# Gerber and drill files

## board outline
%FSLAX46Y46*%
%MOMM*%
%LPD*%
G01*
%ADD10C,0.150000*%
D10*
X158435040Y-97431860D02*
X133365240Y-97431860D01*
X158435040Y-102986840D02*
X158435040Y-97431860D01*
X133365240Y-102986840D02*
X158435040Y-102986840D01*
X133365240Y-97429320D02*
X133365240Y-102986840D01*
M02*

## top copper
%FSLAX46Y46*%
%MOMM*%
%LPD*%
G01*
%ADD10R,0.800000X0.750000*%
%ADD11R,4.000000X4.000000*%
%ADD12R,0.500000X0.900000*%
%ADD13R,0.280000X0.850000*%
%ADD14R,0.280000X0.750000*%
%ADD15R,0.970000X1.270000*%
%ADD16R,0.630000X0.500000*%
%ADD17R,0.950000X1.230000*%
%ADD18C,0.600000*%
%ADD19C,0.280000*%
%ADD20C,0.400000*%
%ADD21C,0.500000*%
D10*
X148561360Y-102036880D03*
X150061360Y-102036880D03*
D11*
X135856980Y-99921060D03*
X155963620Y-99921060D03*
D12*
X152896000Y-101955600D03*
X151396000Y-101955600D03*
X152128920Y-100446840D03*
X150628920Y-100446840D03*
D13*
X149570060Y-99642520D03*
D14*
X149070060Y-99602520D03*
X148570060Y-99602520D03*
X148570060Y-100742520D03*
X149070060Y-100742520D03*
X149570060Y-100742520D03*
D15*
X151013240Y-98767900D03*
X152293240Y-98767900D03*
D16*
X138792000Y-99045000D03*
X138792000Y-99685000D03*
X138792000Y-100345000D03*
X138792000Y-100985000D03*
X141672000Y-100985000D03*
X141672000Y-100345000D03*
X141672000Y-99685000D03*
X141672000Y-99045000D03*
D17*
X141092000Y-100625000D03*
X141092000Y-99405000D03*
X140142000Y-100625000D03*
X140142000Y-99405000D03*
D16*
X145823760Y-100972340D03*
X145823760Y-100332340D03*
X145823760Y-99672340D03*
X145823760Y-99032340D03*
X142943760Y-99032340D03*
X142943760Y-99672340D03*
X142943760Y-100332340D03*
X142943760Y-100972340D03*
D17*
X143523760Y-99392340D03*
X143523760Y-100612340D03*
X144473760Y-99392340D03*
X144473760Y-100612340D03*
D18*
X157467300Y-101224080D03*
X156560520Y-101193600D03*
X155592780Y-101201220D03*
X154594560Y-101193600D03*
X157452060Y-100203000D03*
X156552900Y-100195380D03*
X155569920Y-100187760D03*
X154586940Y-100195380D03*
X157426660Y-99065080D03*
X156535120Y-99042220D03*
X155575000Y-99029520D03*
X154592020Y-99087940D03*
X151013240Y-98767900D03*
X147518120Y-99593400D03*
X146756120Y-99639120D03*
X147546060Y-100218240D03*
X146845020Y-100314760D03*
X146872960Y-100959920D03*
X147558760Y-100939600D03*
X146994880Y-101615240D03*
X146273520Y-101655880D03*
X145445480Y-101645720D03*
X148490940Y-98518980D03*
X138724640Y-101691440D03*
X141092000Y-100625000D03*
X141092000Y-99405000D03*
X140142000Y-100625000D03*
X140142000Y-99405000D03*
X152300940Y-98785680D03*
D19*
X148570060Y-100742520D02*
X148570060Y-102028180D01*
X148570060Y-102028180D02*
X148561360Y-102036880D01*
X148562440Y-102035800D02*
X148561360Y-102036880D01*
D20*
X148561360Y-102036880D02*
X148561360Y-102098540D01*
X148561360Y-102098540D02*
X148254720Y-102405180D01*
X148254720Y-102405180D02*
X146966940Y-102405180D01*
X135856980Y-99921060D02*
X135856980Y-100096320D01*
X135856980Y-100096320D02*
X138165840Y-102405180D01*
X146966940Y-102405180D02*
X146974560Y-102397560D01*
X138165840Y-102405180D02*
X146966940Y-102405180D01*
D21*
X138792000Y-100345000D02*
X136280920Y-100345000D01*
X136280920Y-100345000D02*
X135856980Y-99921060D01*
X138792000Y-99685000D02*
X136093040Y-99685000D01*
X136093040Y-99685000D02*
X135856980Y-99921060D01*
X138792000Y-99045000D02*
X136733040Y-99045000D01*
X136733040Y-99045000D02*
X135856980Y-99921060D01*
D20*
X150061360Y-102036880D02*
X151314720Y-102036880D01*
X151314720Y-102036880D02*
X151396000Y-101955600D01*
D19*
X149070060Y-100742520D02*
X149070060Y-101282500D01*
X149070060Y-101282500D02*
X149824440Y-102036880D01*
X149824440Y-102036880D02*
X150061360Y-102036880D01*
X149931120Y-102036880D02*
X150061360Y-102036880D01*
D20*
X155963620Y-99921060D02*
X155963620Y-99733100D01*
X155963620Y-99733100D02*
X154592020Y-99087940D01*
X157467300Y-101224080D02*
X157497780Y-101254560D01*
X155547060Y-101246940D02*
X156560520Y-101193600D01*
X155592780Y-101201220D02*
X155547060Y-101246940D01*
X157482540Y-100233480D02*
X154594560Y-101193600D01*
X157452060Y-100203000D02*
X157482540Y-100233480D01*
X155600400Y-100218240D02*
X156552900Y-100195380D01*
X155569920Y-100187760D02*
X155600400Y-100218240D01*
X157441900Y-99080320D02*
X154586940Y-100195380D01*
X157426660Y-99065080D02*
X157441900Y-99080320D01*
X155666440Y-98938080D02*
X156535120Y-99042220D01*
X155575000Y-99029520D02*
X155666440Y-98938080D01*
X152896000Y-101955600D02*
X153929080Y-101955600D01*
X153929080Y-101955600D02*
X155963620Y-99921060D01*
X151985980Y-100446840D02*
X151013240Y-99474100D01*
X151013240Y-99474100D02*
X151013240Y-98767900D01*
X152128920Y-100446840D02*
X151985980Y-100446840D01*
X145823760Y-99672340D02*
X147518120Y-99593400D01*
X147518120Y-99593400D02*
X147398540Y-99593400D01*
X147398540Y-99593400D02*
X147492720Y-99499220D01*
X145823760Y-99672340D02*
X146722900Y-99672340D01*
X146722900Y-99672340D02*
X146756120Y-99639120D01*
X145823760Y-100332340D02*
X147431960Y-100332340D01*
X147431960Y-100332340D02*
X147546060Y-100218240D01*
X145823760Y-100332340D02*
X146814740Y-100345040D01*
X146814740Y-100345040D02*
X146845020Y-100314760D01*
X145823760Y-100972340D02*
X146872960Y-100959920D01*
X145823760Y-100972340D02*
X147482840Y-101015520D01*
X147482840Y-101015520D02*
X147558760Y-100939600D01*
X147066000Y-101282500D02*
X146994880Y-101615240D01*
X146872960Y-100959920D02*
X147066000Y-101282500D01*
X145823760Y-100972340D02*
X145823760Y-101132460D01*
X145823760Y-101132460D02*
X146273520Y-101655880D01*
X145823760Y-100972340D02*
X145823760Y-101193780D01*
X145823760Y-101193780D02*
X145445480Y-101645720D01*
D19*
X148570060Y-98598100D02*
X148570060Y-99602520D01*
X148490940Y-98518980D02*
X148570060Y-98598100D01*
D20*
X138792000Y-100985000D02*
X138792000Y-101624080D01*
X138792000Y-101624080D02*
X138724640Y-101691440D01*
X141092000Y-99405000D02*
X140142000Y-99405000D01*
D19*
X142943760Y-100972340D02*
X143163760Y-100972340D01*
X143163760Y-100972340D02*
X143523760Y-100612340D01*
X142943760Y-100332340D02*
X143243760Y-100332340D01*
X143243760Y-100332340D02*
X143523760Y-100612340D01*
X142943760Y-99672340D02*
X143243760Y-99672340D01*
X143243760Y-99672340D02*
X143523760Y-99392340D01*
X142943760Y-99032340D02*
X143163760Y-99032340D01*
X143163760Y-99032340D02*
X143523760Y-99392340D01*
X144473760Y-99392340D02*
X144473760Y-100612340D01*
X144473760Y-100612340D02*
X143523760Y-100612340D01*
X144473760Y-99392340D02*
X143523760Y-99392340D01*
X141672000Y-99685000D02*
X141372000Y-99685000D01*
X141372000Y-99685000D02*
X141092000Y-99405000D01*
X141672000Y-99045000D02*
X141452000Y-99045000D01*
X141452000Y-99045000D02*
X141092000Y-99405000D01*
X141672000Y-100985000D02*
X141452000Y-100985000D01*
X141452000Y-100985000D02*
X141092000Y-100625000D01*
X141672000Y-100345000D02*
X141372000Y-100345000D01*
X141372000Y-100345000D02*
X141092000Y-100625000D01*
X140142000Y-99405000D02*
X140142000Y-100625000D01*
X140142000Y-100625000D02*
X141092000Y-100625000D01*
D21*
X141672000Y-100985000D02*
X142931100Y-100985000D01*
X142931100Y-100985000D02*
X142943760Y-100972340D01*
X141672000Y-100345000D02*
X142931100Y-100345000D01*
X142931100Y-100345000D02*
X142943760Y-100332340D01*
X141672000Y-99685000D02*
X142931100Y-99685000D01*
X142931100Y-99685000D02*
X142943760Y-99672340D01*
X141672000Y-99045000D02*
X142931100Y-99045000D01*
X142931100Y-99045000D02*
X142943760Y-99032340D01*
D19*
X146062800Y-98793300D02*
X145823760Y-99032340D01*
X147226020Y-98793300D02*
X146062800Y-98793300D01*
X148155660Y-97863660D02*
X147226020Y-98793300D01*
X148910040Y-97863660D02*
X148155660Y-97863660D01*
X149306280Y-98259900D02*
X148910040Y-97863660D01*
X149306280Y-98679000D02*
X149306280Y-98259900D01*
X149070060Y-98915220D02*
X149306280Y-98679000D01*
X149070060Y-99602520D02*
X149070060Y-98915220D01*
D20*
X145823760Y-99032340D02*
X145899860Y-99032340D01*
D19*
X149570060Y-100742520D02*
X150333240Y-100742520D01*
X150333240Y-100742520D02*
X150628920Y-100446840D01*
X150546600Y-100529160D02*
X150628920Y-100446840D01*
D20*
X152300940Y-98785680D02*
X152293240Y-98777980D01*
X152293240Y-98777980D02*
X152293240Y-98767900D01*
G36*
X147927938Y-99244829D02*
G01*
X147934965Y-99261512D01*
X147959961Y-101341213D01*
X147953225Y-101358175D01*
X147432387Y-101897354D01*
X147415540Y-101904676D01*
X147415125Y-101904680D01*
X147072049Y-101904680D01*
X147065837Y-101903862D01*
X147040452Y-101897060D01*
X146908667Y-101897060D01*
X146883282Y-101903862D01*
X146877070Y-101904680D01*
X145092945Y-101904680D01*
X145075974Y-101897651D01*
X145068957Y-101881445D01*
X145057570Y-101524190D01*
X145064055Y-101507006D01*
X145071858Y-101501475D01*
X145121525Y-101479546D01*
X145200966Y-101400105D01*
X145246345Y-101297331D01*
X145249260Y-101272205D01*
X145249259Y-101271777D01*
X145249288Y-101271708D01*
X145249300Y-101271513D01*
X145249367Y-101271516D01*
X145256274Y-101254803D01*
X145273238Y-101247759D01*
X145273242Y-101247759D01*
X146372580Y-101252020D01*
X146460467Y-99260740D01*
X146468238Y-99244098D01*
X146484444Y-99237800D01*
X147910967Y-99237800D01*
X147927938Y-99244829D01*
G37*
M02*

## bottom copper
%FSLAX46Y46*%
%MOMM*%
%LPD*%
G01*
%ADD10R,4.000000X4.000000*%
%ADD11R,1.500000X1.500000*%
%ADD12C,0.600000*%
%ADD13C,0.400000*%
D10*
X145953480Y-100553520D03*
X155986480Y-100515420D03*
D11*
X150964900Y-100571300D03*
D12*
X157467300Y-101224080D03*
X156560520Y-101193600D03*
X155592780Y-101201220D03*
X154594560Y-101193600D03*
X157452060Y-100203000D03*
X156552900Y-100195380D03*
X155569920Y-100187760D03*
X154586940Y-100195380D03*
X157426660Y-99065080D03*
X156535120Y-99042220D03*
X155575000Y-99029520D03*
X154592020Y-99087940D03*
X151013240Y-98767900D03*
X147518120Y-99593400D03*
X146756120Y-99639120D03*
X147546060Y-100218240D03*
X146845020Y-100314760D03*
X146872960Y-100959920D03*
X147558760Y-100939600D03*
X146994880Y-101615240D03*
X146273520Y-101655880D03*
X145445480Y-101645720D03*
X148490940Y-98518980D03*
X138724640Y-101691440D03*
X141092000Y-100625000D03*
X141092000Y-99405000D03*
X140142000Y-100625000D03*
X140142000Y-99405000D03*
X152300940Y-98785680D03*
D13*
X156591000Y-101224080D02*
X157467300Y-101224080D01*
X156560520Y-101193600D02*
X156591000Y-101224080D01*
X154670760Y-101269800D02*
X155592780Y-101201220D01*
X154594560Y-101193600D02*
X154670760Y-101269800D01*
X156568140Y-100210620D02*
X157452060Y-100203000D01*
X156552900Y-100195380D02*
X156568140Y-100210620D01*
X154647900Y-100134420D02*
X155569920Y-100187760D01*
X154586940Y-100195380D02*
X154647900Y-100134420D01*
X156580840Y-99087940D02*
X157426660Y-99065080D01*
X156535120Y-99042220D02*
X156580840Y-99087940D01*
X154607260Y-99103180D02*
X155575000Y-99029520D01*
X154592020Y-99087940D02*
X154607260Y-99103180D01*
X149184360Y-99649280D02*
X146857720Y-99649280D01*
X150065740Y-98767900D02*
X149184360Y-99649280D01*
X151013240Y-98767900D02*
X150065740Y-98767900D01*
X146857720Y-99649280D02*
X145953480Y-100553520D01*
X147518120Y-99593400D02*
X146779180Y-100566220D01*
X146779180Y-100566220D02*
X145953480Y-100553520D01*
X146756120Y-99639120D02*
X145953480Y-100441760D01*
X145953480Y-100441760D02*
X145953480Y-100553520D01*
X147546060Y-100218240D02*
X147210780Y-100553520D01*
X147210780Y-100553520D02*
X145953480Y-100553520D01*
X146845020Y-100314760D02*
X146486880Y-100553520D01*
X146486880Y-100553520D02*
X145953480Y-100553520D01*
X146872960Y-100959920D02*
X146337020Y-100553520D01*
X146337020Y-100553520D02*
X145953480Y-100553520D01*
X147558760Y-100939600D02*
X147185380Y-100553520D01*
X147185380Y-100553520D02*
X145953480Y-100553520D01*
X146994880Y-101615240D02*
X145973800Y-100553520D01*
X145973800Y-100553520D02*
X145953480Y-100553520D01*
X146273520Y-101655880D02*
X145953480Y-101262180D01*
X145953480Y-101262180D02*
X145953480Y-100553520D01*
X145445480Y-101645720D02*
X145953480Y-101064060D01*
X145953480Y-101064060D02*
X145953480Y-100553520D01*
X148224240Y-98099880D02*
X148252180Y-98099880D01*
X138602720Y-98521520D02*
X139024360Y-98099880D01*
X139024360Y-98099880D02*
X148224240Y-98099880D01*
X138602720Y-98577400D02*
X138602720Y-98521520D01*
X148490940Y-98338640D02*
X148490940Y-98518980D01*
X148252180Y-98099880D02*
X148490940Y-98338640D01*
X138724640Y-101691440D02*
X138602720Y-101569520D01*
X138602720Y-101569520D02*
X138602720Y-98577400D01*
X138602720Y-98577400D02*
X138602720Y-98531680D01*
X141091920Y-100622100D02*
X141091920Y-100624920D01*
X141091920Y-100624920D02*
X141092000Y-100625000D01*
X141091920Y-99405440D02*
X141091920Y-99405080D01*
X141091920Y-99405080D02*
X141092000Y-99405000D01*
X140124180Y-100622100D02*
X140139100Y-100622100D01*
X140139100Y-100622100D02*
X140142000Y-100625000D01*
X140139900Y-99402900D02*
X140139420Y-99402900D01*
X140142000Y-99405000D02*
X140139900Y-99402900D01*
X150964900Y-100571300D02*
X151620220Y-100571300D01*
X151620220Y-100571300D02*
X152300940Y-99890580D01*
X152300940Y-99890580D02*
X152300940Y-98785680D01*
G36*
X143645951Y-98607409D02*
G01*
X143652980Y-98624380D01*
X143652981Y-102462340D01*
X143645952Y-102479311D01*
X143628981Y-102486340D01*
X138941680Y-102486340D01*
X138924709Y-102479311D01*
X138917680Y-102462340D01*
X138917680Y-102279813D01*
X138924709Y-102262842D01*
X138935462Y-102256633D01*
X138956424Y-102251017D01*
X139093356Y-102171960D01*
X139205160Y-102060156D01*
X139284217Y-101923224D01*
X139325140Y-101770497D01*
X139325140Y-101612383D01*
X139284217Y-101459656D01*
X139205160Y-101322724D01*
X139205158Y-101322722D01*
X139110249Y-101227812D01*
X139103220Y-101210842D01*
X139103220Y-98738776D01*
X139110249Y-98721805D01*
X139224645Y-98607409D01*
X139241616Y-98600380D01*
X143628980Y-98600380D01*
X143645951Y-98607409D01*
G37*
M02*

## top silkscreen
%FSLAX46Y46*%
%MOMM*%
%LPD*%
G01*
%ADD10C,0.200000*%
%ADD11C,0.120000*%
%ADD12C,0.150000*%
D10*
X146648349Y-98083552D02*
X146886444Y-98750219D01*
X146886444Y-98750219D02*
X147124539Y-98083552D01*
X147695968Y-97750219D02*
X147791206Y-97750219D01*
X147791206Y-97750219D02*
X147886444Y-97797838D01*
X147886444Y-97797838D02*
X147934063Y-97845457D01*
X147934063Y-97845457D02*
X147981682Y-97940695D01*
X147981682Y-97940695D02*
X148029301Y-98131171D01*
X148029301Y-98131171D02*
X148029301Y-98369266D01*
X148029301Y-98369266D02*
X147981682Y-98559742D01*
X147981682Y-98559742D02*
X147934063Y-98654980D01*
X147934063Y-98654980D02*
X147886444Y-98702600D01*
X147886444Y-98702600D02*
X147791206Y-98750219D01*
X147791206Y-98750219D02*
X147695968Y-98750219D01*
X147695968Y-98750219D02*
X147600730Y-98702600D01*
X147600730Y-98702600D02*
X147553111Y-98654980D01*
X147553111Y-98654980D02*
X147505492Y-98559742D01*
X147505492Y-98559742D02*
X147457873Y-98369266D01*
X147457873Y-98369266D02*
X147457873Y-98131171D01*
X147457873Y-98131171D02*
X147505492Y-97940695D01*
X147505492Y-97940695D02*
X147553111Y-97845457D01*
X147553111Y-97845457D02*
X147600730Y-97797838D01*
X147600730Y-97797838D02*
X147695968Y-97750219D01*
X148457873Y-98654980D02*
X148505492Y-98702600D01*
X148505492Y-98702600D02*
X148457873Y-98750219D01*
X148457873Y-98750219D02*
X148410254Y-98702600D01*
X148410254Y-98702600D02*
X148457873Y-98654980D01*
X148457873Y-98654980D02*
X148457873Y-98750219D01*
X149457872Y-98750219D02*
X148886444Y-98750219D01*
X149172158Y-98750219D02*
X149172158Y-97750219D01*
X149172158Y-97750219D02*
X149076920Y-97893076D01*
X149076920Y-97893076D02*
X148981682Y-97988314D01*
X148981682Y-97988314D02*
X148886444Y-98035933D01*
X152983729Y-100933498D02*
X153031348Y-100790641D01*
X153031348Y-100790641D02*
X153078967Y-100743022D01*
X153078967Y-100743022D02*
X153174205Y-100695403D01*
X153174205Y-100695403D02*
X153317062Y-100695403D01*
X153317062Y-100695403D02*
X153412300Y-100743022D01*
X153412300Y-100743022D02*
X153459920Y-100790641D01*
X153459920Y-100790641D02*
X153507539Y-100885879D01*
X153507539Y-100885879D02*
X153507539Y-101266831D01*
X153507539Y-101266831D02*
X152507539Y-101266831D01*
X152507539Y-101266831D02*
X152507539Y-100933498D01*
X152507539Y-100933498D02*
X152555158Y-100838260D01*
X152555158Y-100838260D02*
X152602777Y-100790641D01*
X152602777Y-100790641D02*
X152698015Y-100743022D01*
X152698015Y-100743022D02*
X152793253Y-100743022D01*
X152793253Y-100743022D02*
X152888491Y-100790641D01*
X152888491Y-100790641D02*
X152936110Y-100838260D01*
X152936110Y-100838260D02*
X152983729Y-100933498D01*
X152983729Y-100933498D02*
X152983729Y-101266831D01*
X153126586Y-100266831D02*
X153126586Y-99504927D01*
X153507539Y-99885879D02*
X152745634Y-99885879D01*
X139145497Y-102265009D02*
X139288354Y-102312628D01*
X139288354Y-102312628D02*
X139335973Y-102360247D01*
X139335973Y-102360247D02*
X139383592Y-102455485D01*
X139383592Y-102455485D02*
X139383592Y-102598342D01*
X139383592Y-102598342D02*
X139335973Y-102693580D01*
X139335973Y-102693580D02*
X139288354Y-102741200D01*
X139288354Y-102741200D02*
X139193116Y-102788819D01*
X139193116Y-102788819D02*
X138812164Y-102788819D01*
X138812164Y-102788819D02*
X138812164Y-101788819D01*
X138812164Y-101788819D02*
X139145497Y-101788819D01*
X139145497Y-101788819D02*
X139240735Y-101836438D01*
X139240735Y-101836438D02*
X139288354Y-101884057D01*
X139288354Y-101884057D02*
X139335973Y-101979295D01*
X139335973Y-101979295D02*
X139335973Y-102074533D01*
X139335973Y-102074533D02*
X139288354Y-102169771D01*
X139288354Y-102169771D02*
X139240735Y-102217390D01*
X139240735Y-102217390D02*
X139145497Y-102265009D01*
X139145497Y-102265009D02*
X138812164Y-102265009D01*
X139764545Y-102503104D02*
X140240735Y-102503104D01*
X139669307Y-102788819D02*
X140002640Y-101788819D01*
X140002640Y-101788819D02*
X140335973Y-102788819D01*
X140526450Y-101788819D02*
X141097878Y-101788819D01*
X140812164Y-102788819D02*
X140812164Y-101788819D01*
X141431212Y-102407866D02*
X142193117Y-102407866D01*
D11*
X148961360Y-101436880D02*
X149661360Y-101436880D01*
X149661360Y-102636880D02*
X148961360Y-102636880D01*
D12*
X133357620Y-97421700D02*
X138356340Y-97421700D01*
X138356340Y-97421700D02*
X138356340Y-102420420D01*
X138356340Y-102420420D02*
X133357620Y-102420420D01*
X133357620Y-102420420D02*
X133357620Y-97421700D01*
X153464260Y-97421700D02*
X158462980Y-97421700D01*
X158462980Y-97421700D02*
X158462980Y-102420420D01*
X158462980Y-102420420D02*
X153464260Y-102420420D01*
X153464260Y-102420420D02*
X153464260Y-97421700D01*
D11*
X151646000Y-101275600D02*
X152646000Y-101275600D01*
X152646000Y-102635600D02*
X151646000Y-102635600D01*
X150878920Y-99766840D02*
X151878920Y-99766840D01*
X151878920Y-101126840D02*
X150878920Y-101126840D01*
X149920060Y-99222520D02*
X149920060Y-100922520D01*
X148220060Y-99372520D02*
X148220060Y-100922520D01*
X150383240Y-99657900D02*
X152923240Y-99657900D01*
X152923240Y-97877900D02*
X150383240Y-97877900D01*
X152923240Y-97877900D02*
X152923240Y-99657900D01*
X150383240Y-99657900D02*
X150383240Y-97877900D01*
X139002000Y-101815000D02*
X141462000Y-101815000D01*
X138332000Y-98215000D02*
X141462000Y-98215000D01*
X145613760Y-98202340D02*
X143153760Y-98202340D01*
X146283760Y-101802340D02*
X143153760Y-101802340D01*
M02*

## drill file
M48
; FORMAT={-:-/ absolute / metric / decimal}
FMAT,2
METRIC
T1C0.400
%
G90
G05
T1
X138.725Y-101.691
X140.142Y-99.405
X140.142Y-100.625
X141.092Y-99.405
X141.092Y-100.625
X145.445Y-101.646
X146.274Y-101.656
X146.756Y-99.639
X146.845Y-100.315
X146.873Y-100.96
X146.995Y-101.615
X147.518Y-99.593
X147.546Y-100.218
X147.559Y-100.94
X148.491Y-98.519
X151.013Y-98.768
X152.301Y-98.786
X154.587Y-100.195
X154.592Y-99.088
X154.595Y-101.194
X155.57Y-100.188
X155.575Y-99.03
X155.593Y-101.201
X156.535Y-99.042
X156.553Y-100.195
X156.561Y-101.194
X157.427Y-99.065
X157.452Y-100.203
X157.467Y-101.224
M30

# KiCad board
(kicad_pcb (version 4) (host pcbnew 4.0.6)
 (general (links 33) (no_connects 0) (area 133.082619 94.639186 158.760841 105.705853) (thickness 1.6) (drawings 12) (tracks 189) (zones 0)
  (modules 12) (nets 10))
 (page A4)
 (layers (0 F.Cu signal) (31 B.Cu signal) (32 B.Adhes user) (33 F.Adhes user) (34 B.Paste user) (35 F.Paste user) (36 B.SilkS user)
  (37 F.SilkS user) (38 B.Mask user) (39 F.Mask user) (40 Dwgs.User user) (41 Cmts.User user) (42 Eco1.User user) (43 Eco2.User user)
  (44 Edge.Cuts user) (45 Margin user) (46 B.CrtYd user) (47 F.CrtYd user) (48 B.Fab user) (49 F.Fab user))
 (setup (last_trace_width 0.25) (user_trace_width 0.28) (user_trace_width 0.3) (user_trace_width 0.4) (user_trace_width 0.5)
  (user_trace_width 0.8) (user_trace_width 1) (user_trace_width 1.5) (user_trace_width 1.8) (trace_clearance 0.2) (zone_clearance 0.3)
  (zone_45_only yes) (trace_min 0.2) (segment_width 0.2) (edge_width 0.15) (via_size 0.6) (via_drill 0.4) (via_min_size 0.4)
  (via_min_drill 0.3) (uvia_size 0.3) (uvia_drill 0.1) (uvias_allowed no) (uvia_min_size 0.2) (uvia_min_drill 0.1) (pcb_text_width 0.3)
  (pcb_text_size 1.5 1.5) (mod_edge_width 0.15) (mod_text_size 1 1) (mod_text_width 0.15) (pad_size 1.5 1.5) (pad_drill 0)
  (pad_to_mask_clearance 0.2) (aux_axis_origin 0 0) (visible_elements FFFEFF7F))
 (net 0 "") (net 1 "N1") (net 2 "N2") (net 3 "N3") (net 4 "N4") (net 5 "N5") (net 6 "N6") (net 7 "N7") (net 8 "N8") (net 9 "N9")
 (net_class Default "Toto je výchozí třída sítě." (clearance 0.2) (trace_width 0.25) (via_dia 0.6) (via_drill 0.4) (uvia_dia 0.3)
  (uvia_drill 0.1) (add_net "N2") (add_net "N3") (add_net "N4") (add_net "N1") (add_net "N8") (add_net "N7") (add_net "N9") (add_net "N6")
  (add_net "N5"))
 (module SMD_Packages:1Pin (layer B.Cu) (at 145.95348 100.55352)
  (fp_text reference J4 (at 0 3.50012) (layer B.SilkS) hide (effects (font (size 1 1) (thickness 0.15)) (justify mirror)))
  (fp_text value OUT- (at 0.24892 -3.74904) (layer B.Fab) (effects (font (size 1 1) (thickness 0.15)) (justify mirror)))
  (pad 1 smd rect (at 0 0) (size 4 4) (layers B.Cu B.Paste B.Mask) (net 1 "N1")))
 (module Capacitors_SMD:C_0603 (layer F.Cu) (at 149.31136 102.03688)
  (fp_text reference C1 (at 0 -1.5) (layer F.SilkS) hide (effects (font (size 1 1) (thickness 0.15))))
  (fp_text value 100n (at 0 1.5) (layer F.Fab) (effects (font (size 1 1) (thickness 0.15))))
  (fp_line (start -0.35 -0.6) (end 0.35 -0.6) (layer F.SilkS) (width 0.12))
  (fp_line (start 0.35 0.6) (end -0.35 0.6) (layer F.SilkS) (width 0.12))
  (pad 1 smd rect (at -0.75 0) (size 0.8 0.75) (layers F.Cu F.Paste F.Mask) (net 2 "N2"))
  (pad 2 smd rect (at 0.75 0) (size 0.8 0.75) (layers F.Cu F.Paste F.Mask) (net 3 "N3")))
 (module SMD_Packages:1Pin (layer F.Cu) (at 135.85698 99.92106)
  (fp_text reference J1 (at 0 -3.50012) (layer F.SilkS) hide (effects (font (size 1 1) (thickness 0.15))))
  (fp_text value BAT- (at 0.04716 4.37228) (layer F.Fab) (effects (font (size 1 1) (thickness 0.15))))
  (fp_line (start -2.49936 -2.49936) (end 2.49936 -2.49936) (layer F.SilkS) (width 0.15))
  (fp_line (start 2.49936 -2.49936) (end 2.49936 2.49936) (layer F.SilkS) (width 0.15))
  (fp_line (start 2.49936 2.49936) (end -2.49936 2.49936) (layer F.SilkS) (width 0.15))
  (fp_line (start -2.49936 2.49936) (end -2.49936 -2.49936) (layer F.SilkS) (width 0.15))
  (pad 1 smd rect (at 0 0) (size 4 4) (layers F.Cu F.Paste F.Mask) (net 2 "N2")))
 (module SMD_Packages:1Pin (layer F.Cu) (at 155.96362 99.92106)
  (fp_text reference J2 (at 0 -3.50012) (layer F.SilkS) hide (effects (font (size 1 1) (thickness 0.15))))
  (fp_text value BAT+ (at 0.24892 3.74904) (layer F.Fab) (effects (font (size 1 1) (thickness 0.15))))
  (fp_line (start -2.49936 -2.49936) (end 2.49936 -2.49936) (layer F.SilkS) (width 0.15))
  (fp_line (start 2.49936 -2.49936) (end 2.49936 2.49936) (layer F.SilkS) (width 0.15))
  (fp_line (start 2.49936 2.49936) (end -2.49936 2.49936) (layer F.SilkS) (width 0.15))
  (fp_line (start -2.49936 2.49936) (end -2.49936 -2.49936) (layer F.SilkS) (width 0.15))
  (pad 1 smd rect (at 0 0) (size 4 4) (layers F.Cu F.Paste F.Mask) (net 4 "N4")))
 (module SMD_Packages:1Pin (layer B.Cu) (at 155.98648 100.51542)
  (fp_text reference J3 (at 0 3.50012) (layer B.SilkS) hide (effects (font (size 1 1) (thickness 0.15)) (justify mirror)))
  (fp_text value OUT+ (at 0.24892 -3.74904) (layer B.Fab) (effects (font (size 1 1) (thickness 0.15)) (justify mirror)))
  (pad 1 smd rect (at 0 0) (size 4 4) (layers B.Cu B.Paste B.Mask) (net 4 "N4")))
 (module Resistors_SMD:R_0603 (layer F.Cu) (at 152.146 101.9556 180)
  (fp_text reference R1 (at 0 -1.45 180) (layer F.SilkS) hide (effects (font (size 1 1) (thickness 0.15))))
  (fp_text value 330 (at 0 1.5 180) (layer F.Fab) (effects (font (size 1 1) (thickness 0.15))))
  (fp_line (start 0.5 0.68) (end -0.5 0.68) (layer F.SilkS) (width 0.12))
  (fp_line (start -0.5 -0.68) (end 0.5 -0.68) (layer F.SilkS) (width 0.12))
  (pad 1 smd rect (at -0.75 0 180) (size 0.5 0.9) (layers F.Cu F.Paste F.Mask) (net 4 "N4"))
  (pad 2 smd rect (at 0.75 0 180) (size 0.5 0.9) (layers F.Cu F.Paste F.Mask) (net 3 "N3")))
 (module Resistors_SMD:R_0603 (layer F.Cu) (at 151.37892 100.44684 180)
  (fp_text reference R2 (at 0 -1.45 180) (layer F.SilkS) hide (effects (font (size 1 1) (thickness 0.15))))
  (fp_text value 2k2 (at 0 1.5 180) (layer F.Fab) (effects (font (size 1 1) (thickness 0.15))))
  (fp_line (start 0.5 0.68) (end -0.5 0.68) (layer F.SilkS) (width 0.12))
  (fp_line (start -0.5 -0.68) (end 0.5 -0.68) (layer F.SilkS) (width 0.12))
  (pad 1 smd rect (at -0.75 0 180) (size 0.5 0.9) (layers F.Cu F.Paste F.Mask) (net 1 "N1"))
  (pad 2 smd rect (at 0.75 0 180) (size 0.5 0.9) (layers F.Cu F.Paste F.Mask) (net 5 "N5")))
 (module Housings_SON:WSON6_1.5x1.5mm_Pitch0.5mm (layer F.Cu) (at 149.07006 100.17252 270)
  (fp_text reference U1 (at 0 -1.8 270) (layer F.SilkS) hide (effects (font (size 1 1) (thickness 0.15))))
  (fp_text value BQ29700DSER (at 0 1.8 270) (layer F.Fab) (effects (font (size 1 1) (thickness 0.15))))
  (fp_line (start -0.95 -0.85) (end 0.75 -0.85) (layer F.SilkS) (width 0.12))
  (fp_line (start -0.8 0.85) (end 0.75 0.85) (layer F.SilkS) (width 0.12))
  (pad 1 smd rect (at -0.53 -0.5 180) (size 0.28 0.85) (layers F.Cu F.Paste F.Mask))
  (pad 2 smd rect (at -0.57 0 180) (size 0.28 0.75) (layers F.Cu F.Paste F.Mask) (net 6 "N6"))
  (pad 3 smd rect (at -0.57 0.5 180) (size 0.28 0.75) (layers F.Cu F.Paste F.Mask) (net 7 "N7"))
  (pad 4 smd rect (at 0.57 0.5 180) (size 0.28 0.75) (layers F.Cu F.Paste F.Mask) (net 2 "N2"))
  (pad 5 smd rect (at 0.57 0 180) (size 0.28 0.75) (layers F.Cu F.Paste F.Mask) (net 3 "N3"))
  (pad 6 smd rect (at 0.57 -0.5 180) (size 0.28 0.75) (layers F.Cu F.Paste F.Mask) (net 5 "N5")))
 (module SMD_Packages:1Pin (layer B.Cu) (at 150.9649 100.5713)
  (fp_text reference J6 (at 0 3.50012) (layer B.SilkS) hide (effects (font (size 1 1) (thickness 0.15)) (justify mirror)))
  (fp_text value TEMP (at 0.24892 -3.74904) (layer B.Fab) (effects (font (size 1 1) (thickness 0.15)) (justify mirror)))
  (pad 1 smd rect (at 0 0) (size 1.5 1.5) (layers B.Cu B.Paste B.Mask) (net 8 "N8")))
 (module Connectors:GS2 (layer F.Cu) (at 151.65324 98.7679 90)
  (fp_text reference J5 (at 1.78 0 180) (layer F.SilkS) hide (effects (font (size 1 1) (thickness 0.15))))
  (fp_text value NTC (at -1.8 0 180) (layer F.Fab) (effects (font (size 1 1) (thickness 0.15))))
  (fp_line (start -0.89 -1.27) (end -0.89 1.27) (layer F.SilkS) (width 0.12))
  (fp_line (start 0.89 1.27) (end 0.89 -1.27) (layer F.SilkS) (width 0.12))
  (fp_line (start 0.89 1.27) (end -0.89 1.27) (layer F.SilkS) (width 0.12))
  (fp_line (start -0.89 -1.27) (end 0.89 -1.27) (layer F.SilkS) (width 0.12))
  (pad 1 smd rect (at 0 -0.64 90) (size 1.27 0.97) (layers F.Cu F.Paste F.Mask) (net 1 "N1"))
  (pad 2 smd rect (at 0 0.64 90) (size 1.27 0.97) (layers F.Cu F.Paste F.Mask) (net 8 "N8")))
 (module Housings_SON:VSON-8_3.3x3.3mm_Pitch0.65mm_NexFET (layer F.Cu) (at 140.232 100.015)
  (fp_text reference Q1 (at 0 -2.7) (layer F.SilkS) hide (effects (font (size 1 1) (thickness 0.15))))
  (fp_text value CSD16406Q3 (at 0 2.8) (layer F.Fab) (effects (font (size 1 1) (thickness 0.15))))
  (fp_line (start -1.23 1.8) (end 1.23 1.8) (layer F.SilkS) (width 0.12))
  (fp_line (start -1.9 -1.8) (end 1.23 -1.8) (layer F.SilkS) (width 0.12))
  (pad 1 smd rect (at -1.44 -0.97) (size 0.63 0.5) (layers F.Cu F.Paste F.Mask) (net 2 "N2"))
  (pad 2 smd rect (at -1.44 -0.33) (size 0.63 0.5) (layers F.Cu F.Paste F.Mask) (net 2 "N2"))
  (pad 3 smd rect (at -1.44 0.33) (size 0.63 0.5) (layers F.Cu F.Paste F.Mask) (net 2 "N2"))
  (pad 4 smd rect (at -1.44 0.97) (size 0.63 0.5) (layers F.Cu F.Paste F.Mask) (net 7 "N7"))
  (pad 5 smd rect (at 1.44 0.97) (size 0.63 0.5) (layers F.Cu F.Paste F.Mask) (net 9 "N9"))
  (pad 5 smd rect (at 1.44 0.33) (size 0.63 0.5) (layers F.Cu F.Paste F.Mask) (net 9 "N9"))
  (pad 5 smd rect (at 1.44 -0.33) (size 0.63 0.5) (layers F.Cu F.Paste F.Mask) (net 9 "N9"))
  (pad 5 smd rect (at 1.44 -0.97) (size 0.63 0.5) (layers F.Cu F.Paste F.Mask) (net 9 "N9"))
  (pad 5 smd rect (at 0.86 0.61) (size 0.95 1.23) (layers F.Cu F.Paste F.Mask) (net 9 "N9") (solder_paste_margin_ratio -0.2))
  (pad 5 smd rect (at 0.86 -0.61) (size 0.95 1.23) (layers F.Cu F.Paste F.Mask) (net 9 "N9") (solder_paste_margin_ratio -0.2))
  (pad 5 smd rect (at -0.09 0.61) (size 0.95 1.23) (layers F.Cu F.Paste F.Mask) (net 9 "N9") (solder_paste_margin_ratio -0.2))
  (pad 5 smd rect (at -0.09 -0.61) (size 0.95 1.23) (layers F.Cu F.Paste F.Mask) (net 9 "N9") (solder_paste_margin_ratio -0.2)))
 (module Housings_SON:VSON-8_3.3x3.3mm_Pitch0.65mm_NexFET (layer F.Cu) (at 144.38376 100.00234 180)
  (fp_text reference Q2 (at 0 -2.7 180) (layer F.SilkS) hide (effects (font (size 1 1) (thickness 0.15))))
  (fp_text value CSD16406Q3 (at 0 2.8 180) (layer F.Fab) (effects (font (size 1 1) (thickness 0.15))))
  (fp_line (start -1.23 1.8) (end 1.23 1.8) (layer F.SilkS) (width 0.12))
  (fp_line (start -1.9 -1.8) (end 1.23 -1.8) (layer F.SilkS) (width 0.12))
  (pad 1 smd rect (at -1.44 -0.97 180) (size 0.63 0.5) (layers F.Cu F.Paste F.Mask) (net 1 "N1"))
  (pad 2 smd rect (at -1.44 -0.33 180) (size 0.63 0.5) (layers F.Cu F.Paste F.Mask) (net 1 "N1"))
  (pad 3 smd rect (at -1.44 0.33 180) (size 0.63 0.5) (layers F.Cu F.Paste F.Mask) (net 1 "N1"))
  (pad 4 smd rect (at -1.44 0.97 180) (size 0.63 0.5) (layers F.Cu F.Paste F.Mask) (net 6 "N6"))
  (pad 5 smd rect (at 1.44 0.97 180) (size 0.63 0.5) (layers F.Cu F.Paste F.Mask) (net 9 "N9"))
  (pad 5 smd rect (at 1.44 0.33 180) (size 0.63 0.5) (layers F.Cu F.Paste F.Mask) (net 9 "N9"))
  (pad 5 smd rect (at 1.44 -0.33 180) (size 0.63 0.5) (layers F.Cu F.Paste F.Mask) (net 9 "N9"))
  (pad 5 smd rect (at 1.44 -0.97 180) (size 0.63 0.5) (layers F.Cu F.Paste F.Mask) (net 9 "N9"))
  (pad 5 smd rect (at 0.86 0.61 180) (size 0.95 1.23) (layers F.Cu F.Paste F.Mask) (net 9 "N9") (solder_paste_margin_ratio -0.2))
  (pad 5 smd rect (at 0.86 -0.61 180) (size 0.95 1.23) (layers F.Cu F.Paste F.Mask) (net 9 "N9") (solder_paste_margin_ratio -0.2))
  (pad 5 smd rect (at -0.09 0.61 180) (size 0.95 1.23) (layers F.Cu F.Paste F.Mask) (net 9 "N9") (solder_paste_margin_ratio -0.2))
  (pad 5 smd rect (at -0.09 -0.61 180) (size 0.95 1.23) (layers F.Cu F.Paste F.Mask) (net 9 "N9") (solder_paste_margin_ratio -0.2)))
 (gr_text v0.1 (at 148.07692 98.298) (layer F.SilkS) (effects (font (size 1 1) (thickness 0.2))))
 (gr_line (start 158.43504 97.43186) (end 133.36524 97.43186) (angle 90) (layer Edge.Cuts) (width 0.15))
 (gr_line (start 158.43504 102.98684) (end 158.43504 97.43186) (angle 90) (layer Edge.Cuts) (width 0.15))
 (gr_line (start 133.36524 102.98684) (end 158.43504 102.98684) (angle 90) (layer Edge.Cuts) (width 0.15))
 (gr_line (start 133.36524 97.42932) (end 133.36524 102.98684) (angle 90) (layer Edge.Cuts) (width 0.15))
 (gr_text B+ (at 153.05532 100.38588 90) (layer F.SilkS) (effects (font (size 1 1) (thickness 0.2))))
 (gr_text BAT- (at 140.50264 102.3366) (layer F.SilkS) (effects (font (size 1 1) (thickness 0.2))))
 (segment (start 148.57006 100.74252) (end 148.57006 102.02818) (width 0.28) (layer F.Cu) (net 2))
 (segment (start 148.57006 102.02818) (end 148.56136 102.03688) (width 0.28) (layer F.Cu) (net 2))
 (segment (start 148.56244 102.0358) (end 148.56136 102.03688) (width 0.28) (layer F.Cu) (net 2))
 (segment (start 148.56136 102.03688) (end 148.56136 102.09854) (width 0.4) (layer F.Cu) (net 2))
 (segment (start 148.56136 102.09854) (end 148.25472 102.40518) (width 0.4) (layer F.Cu) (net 2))
 (segment (start 148.25472 102.40518) (end 146.96694 102.40518) (width 0.4) (layer F.Cu) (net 2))
 (segment (start 135.85698 99.92106) (end 135.85698 100.09632) (width 0.4) (layer F.Cu) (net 2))
 (segment (start 135.85698 100.09632) (end 138.16584 102.40518) (width 0.4) (layer F.Cu) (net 2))
 (segment (start 146.96694 102.40518) (end 146.97456 102.39756) (width 0.4) (layer F.Cu) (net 2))
 (segment (start 138.16584 102.40518) (end 146.96694 102.40518) (width 0.4) (layer F.Cu) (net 2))
 (segment (start 138.792 100.345) (end 136.28092 100.345) (width 0.5) (layer F.Cu) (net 2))
 (segment (start 136.28092 100.345) (end 135.85698 99.92106) (width 0.5) (layer F.Cu) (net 2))
 (segment (start 138.792 99.685) (end 136.09304 99.685) (width 0.5) (layer F.Cu) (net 2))
 (segment (start 136.09304 99.685) (end 135.85698 99.92106) (width 0.5) (layer F.Cu) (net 2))
 (segment (start 138.792 99.045) (end 136.73304 99.045) (width 0.5) (layer F.Cu) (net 2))
 (segment (start 136.73304 99.045) (end 135.85698 99.92106) (width 0.5) (layer F.Cu) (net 2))
 (segment (start 150.06136 102.03688) (end 151.31472 102.03688) (width 0.4) (layer F.Cu) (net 3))
 (segment (start 151.31472 102.03688) (end 151.396 101.9556) (width 0.4) (layer F.Cu) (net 3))
 (segment (start 149.07006 100.74252) (end 149.07006 101.2825) (width 0.28) (layer F.Cu) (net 3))
 (segment (start 149.07006 101.2825) (end 149.82444 102.03688) (width 0.28) (layer F.Cu) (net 3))
 (segment (start 149.82444 102.03688) (end 150.06136 102.03688) (width 0.28) (layer F.Cu) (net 3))
 (segment (start 149.93112 102.03688) (end 150.06136 102.03688) (width 0.28) (layer F.Cu) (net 3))
 (segment (start 155.96362 99.92106) (end 155.96362 99.7331) (width 0.4) (layer F.Cu) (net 4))
 (segment (start 155.96362 99.7331) (end 154.59202 99.08794) (width 0.4) (layer F.Cu) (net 4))
 (segment (start 157.4673 101.22408) (end 157.49778 101.25456) (width 0.4) (layer F.Cu) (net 4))
 (via (at 157.4673 101.22408) (size 0.6) (drill 0.4) (layers F.Cu B.Cu) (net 4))
 (segment (start 156.591 101.22408) (end 157.4673 101.22408) (width 0.4) (layer B.Cu) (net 4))
 (segment (start 156.56052 101.1936) (end 156.591 101.22408) (width 0.4) (layer B.Cu) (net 4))
 (via (at 156.56052 101.1936) (size 0.6) (drill 0.4) (layers F.Cu B.Cu) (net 4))
 (segment (start 155.54706 101.24694) (end 156.56052 101.1936) (width 0.4) (layer F.Cu) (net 4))
 (segment (start 155.59278 101.20122) (end 155.54706 101.24694) (width 0.4) (layer F.Cu) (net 4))
 (via (at 155.59278 101.20122) (size 0.6) (drill 0.4) (layers F.Cu B.Cu) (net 4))
 (segment (start 154.67076 101.2698) (end 155.59278 101.20122) (width 0.4) (layer B.Cu) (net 4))
 (segment (start 154.59456 101.1936) (end 154.67076 101.2698) (width 0.4) (layer B.Cu) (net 4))
 (via (at 154.59456 101.1936) (size 0.6) (drill 0.4) (layers F.Cu B.Cu) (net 4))
 (segment (start 157.48254 100.23348) (end 154.59456 101.1936) (width 0.4) (layer F.Cu) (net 4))
 (segment (start 157.45206 100.203) (end 157.48254 100.23348) (width 0.4) (layer F.Cu) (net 4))
 (via (at 157.45206 100.203) (size 0.6) (drill 0.4) (layers F.Cu B.Cu) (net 4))
 (segment (start 156.56814 100.21062) (end 157.45206 100.203) (width 0.4) (layer B.Cu) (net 4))
 (segment (start 156.5529 100.19538) (end 156.56814 100.21062) (width 0.4) (layer B.Cu) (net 4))
 (via (at 156.5529 100.19538) (size 0.6) (drill 0.4) (layers F.Cu B.Cu) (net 4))
 (segment (start 155.6004 100.21824) (end 156.5529 100.19538) (width 0.4) (layer F.Cu) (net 4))
 (segment (start 155.56992 100.18776) (end 155.6004 100.21824) (width 0.4) (layer F.Cu) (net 4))
 (via (at 155.56992 100.18776) (size 0.6) (drill 0.4) (layers F.Cu B.Cu) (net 4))
 (segment (start 154.6479 100.13442) (end 155.56992 100.18776) (width 0.4) (layer B.Cu) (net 4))
 (segment (start 154.58694 100.19538) (end 154.6479 100.13442) (width 0.4) (layer B.Cu) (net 4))
 (via (at 154.58694 100.19538) (size 0.6) (drill 0.4) (layers F.Cu B.Cu) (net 4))
 (segment (start 157.4419 99.08032) (end 154.58694 100.19538) (width 0.4) (layer F.Cu) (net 4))
 (segment (start 157.42666 99.06508) (end 157.4419 99.08032) (width 0.4) (layer F.Cu) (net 4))
 (via (at 157.42666 99.06508) (size 0.6) (drill 0.4) (layers F.Cu B.Cu) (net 4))
 (segment (start 156.58084 99.08794) (end 157.42666 99.06508) (width 0.4) (layer B.Cu) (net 4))
 (segment (start 156.53512 99.04222) (end 156.58084 99.08794) (width 0.4) (layer B.Cu) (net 4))
 (via (at 156.53512 99.04222) (size 0.6) (drill 0.4) (layers F.Cu B.Cu) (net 4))
 (segment (start 155.66644 98.93808) (end 156.53512 99.04222) (width 0.4) (layer F.Cu) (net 4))
 (segment (start 155.575 99.02952) (end 155.66644 98.93808) (width 0.4) (layer F.Cu) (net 4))
 (via (at 155.575 99.02952) (size 0.6) (drill 0.4) (layers F.Cu B.Cu) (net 4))
 (segment (start 154.60726 99.10318) (end 155.575 99.02952) (width 0.4) (layer B.Cu) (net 4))
 (segment (start 154.59202 99.08794) (end 154.60726 99.10318) (width 0.4) (layer B.Cu) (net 4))
 (via (at 154.59202 99.08794) (size 0.6) (drill 0.4) (layers F.Cu B.Cu) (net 4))
 (segment (start 152.896 101.9556) (end 153.92908 101.9556) (width 0.4) (layer F.Cu) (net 4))
 (segment (start 153.92908 101.9556) (end 155.96362 99.92106) (width 0.4) (layer F.Cu) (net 4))
 (via (at 151.01324 98.7679) (size 0.6) (drill 0.4) (layers F.Cu B.Cu) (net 1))
 (segment (start 151.98598 100.44684) (end 151.01324 99.4741) (width 0.4) (layer F.Cu) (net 1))
 (segment (start 151.01324 99.4741) (end 151.01324 98.7679) (width 0.4) (layer F.Cu) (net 1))
 (segment (start 149.18436 99.64928) (end 146.85772 99.64928) (width 0.4) (layer B.Cu) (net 1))
 (segment (start 150.06574 98.7679) (end 149.18436 99.64928) (width 0.4) (layer B.Cu) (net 1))
 (segment (start 151.01324 98.7679) (end 150.06574 98.7679) (width 0.4) (layer B.Cu) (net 1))
 (segment (start 146.85772 99.64928) (end 145.95348 100.55352) (width 0.4) (layer B.Cu) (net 1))
 (segment (start 152.12892 100.44684) (end 151.98598 100.44684) (width 0.4) (layer F.Cu) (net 1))
 (via (at 147.51812 99.5934) (size 0.6) (drill 0.4) (layers F.Cu B.Cu) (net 1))
 (segment (start 147.51812 99.5934) (end 146.77918 100.56622) (width 0.4) (layer B.Cu) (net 1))
 (segment (start 146.77918 100.56622) (end 145.95348 100.55352) (width 0.4) (layer B.Cu) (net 1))
 (segment (start 145.82376 99.67234) (end 147.51812 99.5934) (width 0.4) (layer F.Cu) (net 1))
 (segment (start 147.51812 99.5934) (end 147.39854 99.5934) (width 0.4) (layer F.Cu) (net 1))
 (segment (start 147.39854 99.5934) (end 147.49272 99.49922) (width 0.4) (layer F.Cu) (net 1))
 (segment (start 145.82376 99.67234) (end 146.7229 99.67234) (width 0.4) (layer F.Cu) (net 1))
 (segment (start 146.75612 99.63912) (end 145.95348 100.44176) (width 0.4) (layer B.Cu) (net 1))
 (via (at 146.75612 99.63912) (size 0.6) (drill 0.4) (layers F.Cu B.Cu) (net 1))
 (segment (start 146.7229 99.67234) (end 146.75612 99.63912) (width 0.4) (layer F.Cu) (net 1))
 (segment (start 145.95348 100.44176) (end 145.95348 100.55352) (width 0.4) (layer B.Cu) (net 1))
 (segment (start 145.82376 100.33234) (end 147.43196 100.33234) (width 0.4) (layer F.Cu) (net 1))
 (segment (start 147.54606 100.21824) (end 147.21078 100.55352) (width 0.4) (layer B.Cu) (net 1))
 (via (at 147.54606 100.21824) (size 0.6) (drill 0.4) (layers F.Cu B.Cu) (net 1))
 (segment (start 147.43196 100.33234) (end 147.54606 100.21824) (width 0.4) (layer F.Cu) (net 1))
 (segment (start 147.21078 100.55352) (end 145.95348 100.55352) (width 0.4) (layer B.Cu) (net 1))
 (segment (start 145.82376 100.33234) (end 146.81474 100.34504) (width 0.4) (layer F.Cu) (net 1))
 (segment (start 146.84502 100.31476) (end 146.48688 100.55352) (width 0.4) (layer B.Cu) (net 1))
 (via (at 146.84502 100.31476) (size 0.6) (drill 0.4) (layers F.Cu B.Cu) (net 1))
 (segment (start 146.81474 100.34504) (end 146.84502 100.31476) (width 0.4) (layer F.Cu) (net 1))
 (segment (start 146.48688 100.55352) (end 145.95348 100.55352) (width 0.4) (layer B.Cu) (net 1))
 (segment (start 145.82376 100.97234) (end 146.87296 100.95992) (width 0.4) (layer F.Cu) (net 1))
 (via (at 146.87296 100.95992) (size 0.6) (drill 0.4) (layers F.Cu B.Cu) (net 1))
 (segment (start 146.87296 100.95992) (end 146.33702 100.55352) (width 0.4) (layer B.Cu) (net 1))
 (segment (start 146.33702 100.55352) (end 145.95348 100.55352) (width 0.4) (layer B.Cu) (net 1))
 (segment (start 145.82376 100.97234) (end 147.48284 101.01552) (width 0.4) (layer F.Cu) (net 1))
 (segment (start 147.55876 100.9396) (end 147.18538 100.55352) (width 0.4) (layer B.Cu) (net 1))
 (via (at 147.55876 100.9396) (size 0.6) (drill 0.4) (layers F.Cu B.Cu) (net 1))
 (segment (start 147.48284 101.01552) (end 147.55876 100.9396) (width 0.4) (layer F.Cu) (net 1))
 (segment (start 147.18538 100.55352) (end 145.95348 100.55352) (width 0.4) (layer B.Cu) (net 1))
 (segment (start 146.99488 101.61524) (end 145.9738 100.55352) (width 0.4) (layer B.Cu) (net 1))
 (via (at 146.99488 101.61524) (size 0.6) (drill 0.4) (layers F.Cu B.Cu) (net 1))
 (segment (start 147.066 101.2825) (end 146.99488 101.61524) (width 0.4) (layer F.Cu) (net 1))
 (segment (start 146.87296 100.95992) (end 147.066 101.2825) (width 0.4) (layer F.Cu) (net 1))
 (segment (start 145.9738 100.55352) (end 145.95348 100.55352) (width 0.4) (layer B.Cu) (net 1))
 (segment (start 145.82376 100.97234) (end 145.82376 101.13246) (width 0.4) (layer F.Cu) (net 1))
 (segment (start 145.82376 101.13246) (end 146.27352 101.65588) (width 0.4) (layer F.Cu) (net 1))
 (segment (start 146.27352 101.65588) (end 145.95348 101.26218) (width 0.4) (layer B.Cu) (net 1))
 (via (at 146.27352 101.65588) (size 0.6) (drill 0.4) (layers F.Cu B.Cu) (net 1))
 (segment (start 145.95348 101.26218) (end 145.95348 100.55352) (width 0.4) (layer B.Cu) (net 1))
 (segment (start 145.82376 100.97234) (end 145.82376 101.19378) (width 0.4) (layer F.Cu) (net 1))
 (segment (start 145.82376 101.19378) (end 145.44548 101.64572) (width 0.4) (layer F.Cu) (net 1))
 (via (at 145.44548 101.64572) (size 0.6) (drill 0.4) (layers F.Cu B.Cu) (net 1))
 (segment (start 145.44548 101.64572) (end 145.95348 101.06406) (width 0.4) (layer B.Cu) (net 1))
 (segment (start 145.95348 101.06406) (end 145.95348 100.55352) (width 0.4) (layer B.Cu) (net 1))
 (segment (start 148.22424 98.09988) (end 148.25218 98.09988) (width 0.4) (layer B.Cu) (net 7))
 (segment (start 138.60272 98.52152) (end 139.02436 98.09988) (width 0.4) (layer B.Cu) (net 7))
 (segment (start 139.02436 98.09988) (end 148.22424 98.09988) (width 0.4) (layer B.Cu) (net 7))
 (segment (start 138.60272 98.5774) (end 138.60272 98.52152) (width 0.4) (layer B.Cu) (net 7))
 (segment (start 148.57006 98.5981) (end 148.57006 99.60252) (width 0.28) (layer F.Cu) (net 7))
 (segment (start 148.49094 98.51898) (end 148.57006 98.5981) (width 0.28) (layer F.Cu) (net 7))
 (via (at 148.49094 98.51898) (size 0.6) (drill 0.4) (layers F.Cu B.Cu) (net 7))
 (segment (start 148.49094 98.33864) (end 148.49094 98.51898) (width 0.4) (layer B.Cu) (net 7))
 (segment (start 148.25218 98.09988) (end 148.49094 98.33864) (width 0.4) (layer B.Cu) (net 7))
 (segment (start 138.792 100.985) (end 138.792 101.62408) (width 0.4) (layer F.Cu) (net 7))
 (segment (start 138.792 101.62408) (end 138.72464 101.69144) (width 0.4) (layer F.Cu) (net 7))
 (via (at 138.72464 101.69144) (size 0.6) (drill 0.4) (layers F.Cu B.Cu) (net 7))
 (segment (start 138.72464 101.69144) (end 138.60272 101.56952) (width 0.4) (layer B.Cu) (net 7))
 (segment (start 138.60272 101.56952) (end 138.60272 98.5774) (width 0.4) (layer B.Cu) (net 7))
 (segment (start 138.60272 98.5774) (end 138.60272 98.53168) (width 0.4) (layer B.Cu) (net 7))
 (via (at 141.092 100.625) (size 0.6) (drill 0.4) (layers F.Cu B.Cu) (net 9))
 (segment (start 141.09192 100.6221) (end 141.09192 100.62492) (width 0.4) (layer B.Cu) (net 9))
 (segment (start 141.09192 100.62492) (end 141.092 100.625) (width 0.4) (layer B.Cu) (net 9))
 (via (at 141.092 99.405) (size 0.6) (drill 0.4) (layers F.Cu B.Cu) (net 9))
 (segment (start 141.09192 99.40544) (end 141.09192 99.40508) (width 0.4) (layer B.Cu) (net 9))
 (segment (start 141.09192 99.40508) (end 141.092 99.405) (width 0.4) (layer B.Cu) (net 9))
 (via (at 140.142 100.625) (size 0.6) (drill 0.4) (layers F.Cu B.Cu) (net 9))
 (segment (start 140.12418 100.6221) (end 140.1391 100.6221) (width 0.4) (layer B.Cu) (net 9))
 (segment (start 140.1391 100.6221) (end 140.142 100.625) (width 0.4) (layer B.Cu) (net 9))
 (segment (start 141.092 99.405) (end 140.142 99.405) (width 0.4) (layer F.Cu) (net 9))
 (via (at 140.142 99.405) (size 0.6) (drill 0.4) (layers F.Cu B.Cu) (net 9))
 (segment (start 140.1399 99.4029) (end 140.13942 99.4029) (width 0.4) (layer B.Cu) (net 9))
 (segment (start 140.142 99.405) (end 140.1399 99.4029) (width 0.4) (layer B.Cu) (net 9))
 (segment (start 142.94376 100.97234) (end 143.16376 100.97234) (width 0.28) (layer F.Cu) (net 9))
 (segment (start 143.16376 100.97234) (end 143.52376 100.61234) (width 0.28) (layer F.Cu) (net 9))
 (segment (start 142.94376 100.33234) (end 143.24376 100.33234) (width 0.28) (layer F.Cu) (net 9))
 (segment (start 143.24376 100.33234) (end 143.52376 100.61234) (width 0.28) (layer F.Cu) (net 9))
 (segment (start 142.94376 99.67234) (end 143.24376 99.67234) (width 0.28) (layer F.Cu) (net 9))
 (segment (start 143.24376 99.67234) (end 143.52376 99.39234) (width 0.28) (layer F.Cu) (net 9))
 (segment (start 142.94376 99.03234) (end 143.16376 99.03234) (width 0.28) (layer F.Cu) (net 9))
 (segment (start 143.16376 99.03234) (end 143.52376 99.39234) (width 0.28) (layer F.Cu) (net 9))
 (segment (start 144.47376 99.39234) (end 144.47376 100.61234) (width 0.28) (layer F.Cu) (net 9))
 (segment (start 144.47376 100.61234) (end 143.52376 100.61234) (width 0.28) (layer F.Cu) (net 9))
 (segment (start 144.47376 99.39234) (end 143.52376 99.39234) (width 0.28) (layer F.Cu) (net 9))
 (segment (start 141.672 99.685) (end 141.372 99.685) (width 0.28) (layer F.Cu) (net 9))
 (segment (start 141.372 99.685) (end 141.092 99.405) (width 0.28) (layer F.Cu) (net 9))
 (segment (start 141.672 99.045) (end 141.452 99.045) (width 0.28) (layer F.Cu) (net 9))
 (segment (start 141.452 99.045) (end 141.092 99.405) (width 0.28) (layer F.Cu) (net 9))
 (segment (start 141.672 100.985) (end 141.452 100.985) (width 0.28) (layer F.Cu) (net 9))
 (segment (start 141.452 100.985) (end 141.092 100.625) (width 0.28) (layer F.Cu) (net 9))
 (segment (start 141.672 100.345) (end 141.372 100.345) (width 0.28) (layer F.Cu) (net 9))
 (segment (start 141.372 100.345) (end 141.092 100.625) (width 0.28) (layer F.Cu) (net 9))
 (segment (start 140.142 99.405) (end 140.142 100.625) (width 0.28) (layer F.Cu) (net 9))
 (segment (start 140.142 100.625) (end 141.092 100.625) (width 0.28) (layer F.Cu) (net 9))
 (segment (start 141.672 100.985) (end 142.9311 100.985) (width 0.5) (layer F.Cu) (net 9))
 (segment (start 142.9311 100.985) (end 142.94376 100.97234) (width 0.5) (layer F.Cu) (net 9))
 (segment (start 141.672 100.345) (end 142.9311 100.345) (width 0.5) (layer F.Cu) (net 9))
 (segment (start 142.9311 100.345) (end 142.94376 100.33234) (width 0.5) (layer F.Cu) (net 9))
 (segment (start 141.672 99.685) (end 142.9311 99.685) (width 0.5) (layer F.Cu) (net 9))
 (segment (start 142.9311 99.685) (end 142.94376 99.67234) (width 0.5) (layer F.Cu) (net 9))
 (segment (start 141.672 99.045) (end 142.9311 99.045) (width 0.5) (layer F.Cu) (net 9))
 (segment (start 142.9311 99.045) (end 142.94376 99.03234) (width 0.5) (layer F.Cu) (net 9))
 (segment (start 146.0628 98.7933) (end 145.82376 99.03234) (width 0.28) (layer F.Cu) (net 6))
 (segment (start 147.22602 98.7933) (end 146.0628 98.7933) (width 0.28) (layer F.Cu) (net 6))
 (segment (start 148.15566 97.86366) (end 147.22602 98.7933) (width 0.28) (layer F.Cu) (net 6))
 (segment (start 148.91004 97.86366) (end 148.15566 97.86366) (width 0.28) (layer F.Cu) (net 6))
 (segment (start 149.30628 98.2599) (end 148.91004 97.86366) (width 0.28) (layer F.Cu) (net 6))
 (segment (start 149.30628 98.679) (end 149.30628 98.2599) (width 0.28) (layer F.Cu) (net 6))
 (segment (start 149.07006 98.91522) (end 149.30628 98.679) (width 0.28) (layer F.Cu) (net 6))
 (segment (start 149.07006 99.60252) (end 149.07006 98.91522) (width 0.28) (layer F.Cu) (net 6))
 (segment (start 145.82376 99.03234) (end 145.89986 99.03234) (width 0.4) (layer F.Cu) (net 6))
 (segment (start 149.57006 100.74252) (end 150.33324 100.74252) (width 0.28) (layer F.Cu) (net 5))
 (segment (start 150.33324 100.74252) (end 150.62892 100.44684) (width 0.28) (layer F.Cu) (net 5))
 (segment (start 150.5466 100.52916) (end 150.62892 100.44684) (width 0.28) (layer F.Cu) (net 5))
 (segment (start 150.9649 100.5713) (end 151.62022 100.5713) (width 0.4) (layer B.Cu) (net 8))
 (segment (start 151.62022 100.5713) (end 152.30094 99.89058) (width 0.4) (layer B.Cu) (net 8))
 (segment (start 152.30094 99.89058) (end 152.30094 98.78568) (width 0.4) (layer B.Cu) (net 8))
 (via (at 152.30094 98.78568) (size 0.6) (drill 0.4) (layers F.Cu B.Cu) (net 8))
 (segment (start 152.30094 98.78568) (end 152.29324 98.77798) (width 0.4) (layer F.Cu) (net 8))
 (segment (start 152.29324 98.77798) (end 152.29324 98.7679) (width 0.4) (layer F.Cu) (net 8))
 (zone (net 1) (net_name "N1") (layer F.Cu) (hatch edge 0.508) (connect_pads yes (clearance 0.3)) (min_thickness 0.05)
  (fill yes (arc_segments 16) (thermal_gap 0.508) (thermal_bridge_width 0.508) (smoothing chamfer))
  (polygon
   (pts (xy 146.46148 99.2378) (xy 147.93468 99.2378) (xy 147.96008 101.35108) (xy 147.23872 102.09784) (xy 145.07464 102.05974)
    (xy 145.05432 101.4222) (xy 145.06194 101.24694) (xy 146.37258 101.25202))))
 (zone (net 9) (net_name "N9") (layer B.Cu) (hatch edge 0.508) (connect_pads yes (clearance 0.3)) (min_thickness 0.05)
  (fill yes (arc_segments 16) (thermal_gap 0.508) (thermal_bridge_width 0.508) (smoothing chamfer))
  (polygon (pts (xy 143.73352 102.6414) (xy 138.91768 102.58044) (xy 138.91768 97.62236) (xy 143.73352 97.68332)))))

